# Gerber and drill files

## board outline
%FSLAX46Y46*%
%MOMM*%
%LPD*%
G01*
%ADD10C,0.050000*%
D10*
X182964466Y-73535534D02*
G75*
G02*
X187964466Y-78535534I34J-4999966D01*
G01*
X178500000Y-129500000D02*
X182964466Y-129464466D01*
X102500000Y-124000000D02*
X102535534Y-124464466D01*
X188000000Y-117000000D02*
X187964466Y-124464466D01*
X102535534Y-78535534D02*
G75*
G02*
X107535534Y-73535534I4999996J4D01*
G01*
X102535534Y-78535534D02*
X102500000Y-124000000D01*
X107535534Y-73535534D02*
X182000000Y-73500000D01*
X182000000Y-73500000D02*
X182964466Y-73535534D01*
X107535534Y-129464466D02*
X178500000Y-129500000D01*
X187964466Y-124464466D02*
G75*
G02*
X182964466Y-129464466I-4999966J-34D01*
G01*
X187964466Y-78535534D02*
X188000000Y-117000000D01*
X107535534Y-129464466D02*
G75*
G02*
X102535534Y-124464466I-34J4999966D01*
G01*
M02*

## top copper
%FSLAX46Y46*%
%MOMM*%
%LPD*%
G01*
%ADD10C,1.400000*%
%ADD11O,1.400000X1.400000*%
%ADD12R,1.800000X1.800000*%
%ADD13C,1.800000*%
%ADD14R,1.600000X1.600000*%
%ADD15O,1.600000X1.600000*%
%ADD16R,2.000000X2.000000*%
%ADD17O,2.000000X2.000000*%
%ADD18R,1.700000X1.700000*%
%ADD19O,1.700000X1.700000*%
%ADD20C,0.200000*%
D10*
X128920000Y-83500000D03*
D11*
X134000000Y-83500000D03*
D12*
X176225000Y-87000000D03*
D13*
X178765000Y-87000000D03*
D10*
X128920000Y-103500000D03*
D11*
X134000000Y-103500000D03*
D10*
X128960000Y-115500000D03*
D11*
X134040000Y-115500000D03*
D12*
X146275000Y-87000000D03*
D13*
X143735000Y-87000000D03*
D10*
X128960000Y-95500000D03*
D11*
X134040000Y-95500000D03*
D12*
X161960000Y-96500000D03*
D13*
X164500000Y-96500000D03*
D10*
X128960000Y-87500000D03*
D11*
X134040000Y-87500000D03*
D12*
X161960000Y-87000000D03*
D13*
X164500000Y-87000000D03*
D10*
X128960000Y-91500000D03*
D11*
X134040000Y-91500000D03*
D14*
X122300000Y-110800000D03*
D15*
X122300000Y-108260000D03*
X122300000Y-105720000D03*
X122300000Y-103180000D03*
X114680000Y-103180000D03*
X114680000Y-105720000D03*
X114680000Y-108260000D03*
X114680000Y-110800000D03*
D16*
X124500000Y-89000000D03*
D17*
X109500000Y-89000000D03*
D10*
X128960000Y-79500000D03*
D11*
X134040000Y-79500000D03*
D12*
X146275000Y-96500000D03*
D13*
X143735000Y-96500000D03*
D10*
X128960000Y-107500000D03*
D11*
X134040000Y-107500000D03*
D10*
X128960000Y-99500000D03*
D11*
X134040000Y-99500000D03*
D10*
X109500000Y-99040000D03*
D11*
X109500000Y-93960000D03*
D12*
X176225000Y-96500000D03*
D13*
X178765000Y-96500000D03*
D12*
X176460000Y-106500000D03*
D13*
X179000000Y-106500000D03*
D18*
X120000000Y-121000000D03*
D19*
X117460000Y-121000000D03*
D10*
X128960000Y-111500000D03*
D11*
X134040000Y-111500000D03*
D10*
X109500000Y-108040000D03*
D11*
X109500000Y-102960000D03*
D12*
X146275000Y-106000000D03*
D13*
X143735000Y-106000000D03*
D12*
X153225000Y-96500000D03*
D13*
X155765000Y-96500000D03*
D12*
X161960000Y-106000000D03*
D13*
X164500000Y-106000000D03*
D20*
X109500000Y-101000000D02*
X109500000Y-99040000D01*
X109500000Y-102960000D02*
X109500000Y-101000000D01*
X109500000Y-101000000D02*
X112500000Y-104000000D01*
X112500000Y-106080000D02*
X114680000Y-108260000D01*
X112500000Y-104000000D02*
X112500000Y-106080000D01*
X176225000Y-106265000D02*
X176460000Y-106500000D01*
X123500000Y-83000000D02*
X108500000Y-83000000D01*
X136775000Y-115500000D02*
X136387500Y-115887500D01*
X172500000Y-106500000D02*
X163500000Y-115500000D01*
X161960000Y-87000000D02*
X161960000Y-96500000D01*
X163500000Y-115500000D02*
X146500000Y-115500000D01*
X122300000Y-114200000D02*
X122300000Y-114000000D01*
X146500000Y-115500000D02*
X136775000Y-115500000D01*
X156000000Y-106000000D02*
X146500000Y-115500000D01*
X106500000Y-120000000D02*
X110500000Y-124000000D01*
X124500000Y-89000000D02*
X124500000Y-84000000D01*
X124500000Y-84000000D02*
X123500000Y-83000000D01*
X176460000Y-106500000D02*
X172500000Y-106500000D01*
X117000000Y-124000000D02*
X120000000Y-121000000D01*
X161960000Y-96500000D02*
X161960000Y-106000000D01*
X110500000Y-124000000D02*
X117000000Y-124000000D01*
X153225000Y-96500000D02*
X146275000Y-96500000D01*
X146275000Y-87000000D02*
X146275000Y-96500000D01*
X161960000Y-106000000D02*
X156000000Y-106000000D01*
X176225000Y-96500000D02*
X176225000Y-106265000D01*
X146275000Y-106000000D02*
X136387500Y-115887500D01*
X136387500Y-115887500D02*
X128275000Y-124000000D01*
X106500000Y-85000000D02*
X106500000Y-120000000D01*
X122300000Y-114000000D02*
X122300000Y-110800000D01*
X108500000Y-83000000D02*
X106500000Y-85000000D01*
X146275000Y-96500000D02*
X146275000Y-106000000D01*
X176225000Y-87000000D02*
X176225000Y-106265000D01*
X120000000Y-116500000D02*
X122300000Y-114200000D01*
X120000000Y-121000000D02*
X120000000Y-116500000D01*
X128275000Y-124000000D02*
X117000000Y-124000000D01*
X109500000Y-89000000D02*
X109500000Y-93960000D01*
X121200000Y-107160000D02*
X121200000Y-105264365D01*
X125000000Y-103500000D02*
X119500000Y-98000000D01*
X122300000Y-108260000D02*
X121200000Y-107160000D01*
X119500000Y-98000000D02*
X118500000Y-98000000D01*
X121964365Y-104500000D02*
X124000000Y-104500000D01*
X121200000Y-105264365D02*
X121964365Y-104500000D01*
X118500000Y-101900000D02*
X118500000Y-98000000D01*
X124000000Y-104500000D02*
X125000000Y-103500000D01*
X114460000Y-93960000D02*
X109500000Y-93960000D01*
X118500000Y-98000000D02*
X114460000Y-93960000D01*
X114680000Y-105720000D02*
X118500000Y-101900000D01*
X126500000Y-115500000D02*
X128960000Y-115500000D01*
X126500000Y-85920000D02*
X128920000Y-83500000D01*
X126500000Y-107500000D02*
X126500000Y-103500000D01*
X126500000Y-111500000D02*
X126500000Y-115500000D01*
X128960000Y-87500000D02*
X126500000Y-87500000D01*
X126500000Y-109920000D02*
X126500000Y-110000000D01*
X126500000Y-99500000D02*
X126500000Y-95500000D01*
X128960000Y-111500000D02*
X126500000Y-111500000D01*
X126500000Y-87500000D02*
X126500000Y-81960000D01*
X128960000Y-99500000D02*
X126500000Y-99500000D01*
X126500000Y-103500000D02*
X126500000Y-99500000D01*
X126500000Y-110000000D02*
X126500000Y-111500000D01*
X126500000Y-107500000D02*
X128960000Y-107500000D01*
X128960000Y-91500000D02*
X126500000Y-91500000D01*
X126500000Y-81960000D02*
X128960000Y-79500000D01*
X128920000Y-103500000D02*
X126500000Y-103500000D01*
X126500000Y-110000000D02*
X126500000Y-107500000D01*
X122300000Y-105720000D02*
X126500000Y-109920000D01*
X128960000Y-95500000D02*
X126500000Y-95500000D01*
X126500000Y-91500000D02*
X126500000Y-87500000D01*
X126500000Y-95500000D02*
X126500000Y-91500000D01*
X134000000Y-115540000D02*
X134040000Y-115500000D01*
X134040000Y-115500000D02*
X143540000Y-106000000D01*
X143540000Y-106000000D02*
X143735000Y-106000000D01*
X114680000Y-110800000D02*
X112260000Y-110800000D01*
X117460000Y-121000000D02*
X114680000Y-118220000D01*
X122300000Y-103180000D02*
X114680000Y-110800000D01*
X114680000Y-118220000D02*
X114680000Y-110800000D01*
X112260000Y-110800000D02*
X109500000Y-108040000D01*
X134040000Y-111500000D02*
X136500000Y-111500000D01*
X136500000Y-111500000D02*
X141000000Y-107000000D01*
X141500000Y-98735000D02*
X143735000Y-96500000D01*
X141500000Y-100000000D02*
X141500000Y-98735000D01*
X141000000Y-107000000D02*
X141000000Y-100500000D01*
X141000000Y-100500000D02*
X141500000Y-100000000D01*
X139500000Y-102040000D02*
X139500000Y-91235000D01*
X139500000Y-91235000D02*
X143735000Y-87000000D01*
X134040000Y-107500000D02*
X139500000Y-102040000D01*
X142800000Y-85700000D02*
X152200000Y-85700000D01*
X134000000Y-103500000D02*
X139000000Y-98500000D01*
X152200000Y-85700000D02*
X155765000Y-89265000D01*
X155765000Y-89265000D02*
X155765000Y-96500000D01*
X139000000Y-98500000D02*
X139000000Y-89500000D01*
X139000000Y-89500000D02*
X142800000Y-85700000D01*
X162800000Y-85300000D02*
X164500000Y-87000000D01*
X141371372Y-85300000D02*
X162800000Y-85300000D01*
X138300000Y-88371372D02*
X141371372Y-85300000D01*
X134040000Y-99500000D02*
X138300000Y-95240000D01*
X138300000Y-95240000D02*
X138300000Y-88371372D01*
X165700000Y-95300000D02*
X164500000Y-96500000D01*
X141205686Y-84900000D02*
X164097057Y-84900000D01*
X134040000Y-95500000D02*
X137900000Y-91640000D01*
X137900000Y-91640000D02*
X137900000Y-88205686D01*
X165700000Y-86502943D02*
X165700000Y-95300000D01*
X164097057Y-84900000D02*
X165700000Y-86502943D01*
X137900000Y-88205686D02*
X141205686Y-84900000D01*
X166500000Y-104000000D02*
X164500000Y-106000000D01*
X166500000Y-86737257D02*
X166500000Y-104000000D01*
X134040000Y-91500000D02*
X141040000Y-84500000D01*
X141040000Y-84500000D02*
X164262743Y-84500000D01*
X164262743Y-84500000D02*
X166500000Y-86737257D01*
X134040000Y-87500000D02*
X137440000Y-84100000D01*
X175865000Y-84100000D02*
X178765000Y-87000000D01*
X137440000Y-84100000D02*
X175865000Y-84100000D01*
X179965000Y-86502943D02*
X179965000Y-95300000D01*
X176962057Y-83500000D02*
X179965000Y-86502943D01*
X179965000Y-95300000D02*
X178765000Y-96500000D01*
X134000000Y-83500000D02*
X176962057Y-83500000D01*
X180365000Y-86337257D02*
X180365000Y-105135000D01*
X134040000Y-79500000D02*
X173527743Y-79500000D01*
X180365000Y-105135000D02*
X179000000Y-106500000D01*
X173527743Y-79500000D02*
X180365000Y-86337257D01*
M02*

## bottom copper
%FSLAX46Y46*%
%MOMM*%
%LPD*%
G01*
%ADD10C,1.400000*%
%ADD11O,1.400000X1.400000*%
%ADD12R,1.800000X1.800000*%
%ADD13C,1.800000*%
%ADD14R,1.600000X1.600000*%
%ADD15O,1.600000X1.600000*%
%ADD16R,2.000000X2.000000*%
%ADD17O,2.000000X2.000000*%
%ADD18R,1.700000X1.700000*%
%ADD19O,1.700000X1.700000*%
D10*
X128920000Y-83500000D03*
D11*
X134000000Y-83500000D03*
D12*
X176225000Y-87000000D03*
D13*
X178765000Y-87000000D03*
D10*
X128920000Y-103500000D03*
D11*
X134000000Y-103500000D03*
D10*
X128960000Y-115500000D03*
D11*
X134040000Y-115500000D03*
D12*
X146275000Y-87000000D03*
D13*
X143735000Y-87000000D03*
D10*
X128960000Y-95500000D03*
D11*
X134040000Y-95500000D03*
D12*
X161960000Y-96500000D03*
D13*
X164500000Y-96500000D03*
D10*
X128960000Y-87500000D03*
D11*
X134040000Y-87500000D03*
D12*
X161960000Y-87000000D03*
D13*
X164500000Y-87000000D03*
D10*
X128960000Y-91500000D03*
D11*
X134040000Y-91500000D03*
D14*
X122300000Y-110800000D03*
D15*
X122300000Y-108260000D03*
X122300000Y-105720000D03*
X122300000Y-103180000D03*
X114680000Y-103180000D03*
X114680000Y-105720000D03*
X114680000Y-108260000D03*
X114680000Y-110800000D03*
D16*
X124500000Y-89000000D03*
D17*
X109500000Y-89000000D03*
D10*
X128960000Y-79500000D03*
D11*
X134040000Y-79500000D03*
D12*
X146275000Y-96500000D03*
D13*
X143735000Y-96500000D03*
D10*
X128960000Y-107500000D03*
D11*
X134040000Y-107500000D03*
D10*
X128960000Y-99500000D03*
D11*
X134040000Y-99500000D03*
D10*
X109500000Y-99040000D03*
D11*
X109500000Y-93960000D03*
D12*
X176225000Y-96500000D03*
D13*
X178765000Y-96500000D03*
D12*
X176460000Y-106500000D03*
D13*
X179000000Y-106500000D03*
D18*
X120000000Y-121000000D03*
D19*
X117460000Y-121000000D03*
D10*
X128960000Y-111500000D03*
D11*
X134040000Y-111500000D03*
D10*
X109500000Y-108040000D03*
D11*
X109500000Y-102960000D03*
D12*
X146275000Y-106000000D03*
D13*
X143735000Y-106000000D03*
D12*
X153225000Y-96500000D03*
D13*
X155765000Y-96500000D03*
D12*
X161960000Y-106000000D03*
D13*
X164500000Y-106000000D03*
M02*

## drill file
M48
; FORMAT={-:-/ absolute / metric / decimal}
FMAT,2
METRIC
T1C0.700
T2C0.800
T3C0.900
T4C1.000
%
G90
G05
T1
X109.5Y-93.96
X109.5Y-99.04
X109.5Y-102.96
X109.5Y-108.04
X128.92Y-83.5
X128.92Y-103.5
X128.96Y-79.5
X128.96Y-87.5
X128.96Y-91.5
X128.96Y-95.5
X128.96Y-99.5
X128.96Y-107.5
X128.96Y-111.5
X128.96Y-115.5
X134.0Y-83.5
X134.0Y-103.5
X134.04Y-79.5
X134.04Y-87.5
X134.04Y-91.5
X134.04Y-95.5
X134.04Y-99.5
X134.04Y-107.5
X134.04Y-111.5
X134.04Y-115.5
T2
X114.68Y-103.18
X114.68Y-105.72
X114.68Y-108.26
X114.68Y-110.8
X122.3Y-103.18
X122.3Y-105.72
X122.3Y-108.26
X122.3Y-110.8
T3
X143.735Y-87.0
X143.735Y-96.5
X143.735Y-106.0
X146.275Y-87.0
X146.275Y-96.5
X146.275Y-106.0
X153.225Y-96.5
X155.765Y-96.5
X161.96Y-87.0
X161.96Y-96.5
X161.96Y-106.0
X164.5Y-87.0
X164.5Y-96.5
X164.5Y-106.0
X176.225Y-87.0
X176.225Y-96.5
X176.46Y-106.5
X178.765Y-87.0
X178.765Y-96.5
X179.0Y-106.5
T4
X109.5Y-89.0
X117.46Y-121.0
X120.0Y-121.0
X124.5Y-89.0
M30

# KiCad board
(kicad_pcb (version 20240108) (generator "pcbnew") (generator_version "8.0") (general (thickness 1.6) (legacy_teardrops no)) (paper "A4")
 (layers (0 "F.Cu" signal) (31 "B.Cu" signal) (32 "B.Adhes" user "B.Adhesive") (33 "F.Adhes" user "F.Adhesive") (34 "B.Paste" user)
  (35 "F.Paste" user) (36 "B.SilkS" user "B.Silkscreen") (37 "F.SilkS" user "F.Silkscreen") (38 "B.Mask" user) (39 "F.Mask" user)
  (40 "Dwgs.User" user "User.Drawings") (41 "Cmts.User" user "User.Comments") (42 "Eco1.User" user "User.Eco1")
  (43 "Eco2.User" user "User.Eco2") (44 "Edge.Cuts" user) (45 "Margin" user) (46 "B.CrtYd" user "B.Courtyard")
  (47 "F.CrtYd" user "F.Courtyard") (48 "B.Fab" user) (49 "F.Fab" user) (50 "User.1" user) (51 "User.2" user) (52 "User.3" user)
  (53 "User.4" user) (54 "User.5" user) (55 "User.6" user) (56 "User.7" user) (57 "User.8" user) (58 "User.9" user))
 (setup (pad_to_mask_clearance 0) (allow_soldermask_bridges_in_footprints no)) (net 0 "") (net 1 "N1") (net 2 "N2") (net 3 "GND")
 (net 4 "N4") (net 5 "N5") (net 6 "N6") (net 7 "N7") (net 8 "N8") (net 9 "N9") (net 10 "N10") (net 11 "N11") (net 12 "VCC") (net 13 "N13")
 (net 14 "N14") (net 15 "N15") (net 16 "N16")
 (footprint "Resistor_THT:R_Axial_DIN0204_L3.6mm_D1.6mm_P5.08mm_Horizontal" (layer "F.Cu") (at 128.92 83.5)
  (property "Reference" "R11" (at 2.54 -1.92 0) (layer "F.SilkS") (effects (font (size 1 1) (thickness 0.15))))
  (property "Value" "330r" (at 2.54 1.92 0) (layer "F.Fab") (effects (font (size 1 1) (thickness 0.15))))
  (pad "1" thru_hole circle (at 0 0) (size 1.4 1.4) (drill 0.7) (layers "*.Cu" "*.Mask") (remove_unused_layers no) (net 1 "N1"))
  (pad "2" thru_hole oval (at 5.08 0) (size 1.4 1.4) (drill 0.7) (layers "*.Cu" "*.Mask") (remove_unused_layers no) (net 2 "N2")))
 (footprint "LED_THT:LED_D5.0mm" (layer "F.Cu") (at 176.225 87)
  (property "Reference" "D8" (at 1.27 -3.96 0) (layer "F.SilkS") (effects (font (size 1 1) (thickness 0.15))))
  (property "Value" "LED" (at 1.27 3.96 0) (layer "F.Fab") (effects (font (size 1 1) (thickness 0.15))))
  (pad "1" thru_hole rect (at 0 0) (size 1.8 1.8) (drill 0.9) (layers "*.Cu" "*.Mask") (remove_unused_layers no) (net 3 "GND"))
  (pad "2" thru_hole circle (at 2.54 0) (size 1.8 1.8) (drill 0.9) (layers "*.Cu" "*.Mask") (remove_unused_layers no) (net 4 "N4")))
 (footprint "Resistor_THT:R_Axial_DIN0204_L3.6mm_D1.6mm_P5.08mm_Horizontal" (layer "F.Cu") (at 128.92 103.5)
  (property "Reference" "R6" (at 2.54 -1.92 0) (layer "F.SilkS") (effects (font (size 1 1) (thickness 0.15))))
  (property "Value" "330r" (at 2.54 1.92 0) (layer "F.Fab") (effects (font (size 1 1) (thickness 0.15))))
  (pad "1" thru_hole circle (at 0 0) (size 1.4 1.4) (drill 0.7) (layers "*.Cu" "*.Mask") (remove_unused_layers no) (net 1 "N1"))
  (pad "2" thru_hole oval (at 5.08 0) (size 1.4 1.4) (drill 0.7) (layers "*.Cu" "*.Mask") (remove_unused_layers no) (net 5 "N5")))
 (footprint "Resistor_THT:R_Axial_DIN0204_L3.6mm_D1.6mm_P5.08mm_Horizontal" (layer "F.Cu") (at 128.96 115.5)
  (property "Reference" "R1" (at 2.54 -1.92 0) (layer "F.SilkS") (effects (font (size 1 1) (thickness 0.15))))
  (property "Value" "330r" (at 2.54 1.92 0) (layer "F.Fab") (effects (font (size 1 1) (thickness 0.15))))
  (pad "1" thru_hole circle (at 0 0) (size 1.4 1.4) (drill 0.7) (layers "*.Cu" "*.Mask") (remove_unused_layers no) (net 1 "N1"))
  (pad "2" thru_hole oval (at 5.08 0) (size 1.4 1.4) (drill 0.7) (layers "*.Cu" "*.Mask") (remove_unused_layers no) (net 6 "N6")))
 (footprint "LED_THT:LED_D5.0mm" (layer "F.Cu") (at 146.275 87 180)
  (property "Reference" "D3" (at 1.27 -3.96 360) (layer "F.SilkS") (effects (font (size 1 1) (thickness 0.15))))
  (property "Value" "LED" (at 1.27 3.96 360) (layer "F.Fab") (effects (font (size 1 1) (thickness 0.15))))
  (pad "1" thru_hole rect (at 0 0 180) (size 1.8 1.8) (drill 0.9) (layers "*.Cu" "*.Mask") (remove_unused_layers no) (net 3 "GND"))
  (pad "2" thru_hole circle (at 2.54 0 180) (size 1.8 1.8) (drill 0.9) (layers "*.Cu" "*.Mask") (remove_unused_layers no) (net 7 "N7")))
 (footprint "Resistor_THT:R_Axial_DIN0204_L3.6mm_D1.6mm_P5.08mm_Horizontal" (layer "F.Cu") (at 128.96 95.5)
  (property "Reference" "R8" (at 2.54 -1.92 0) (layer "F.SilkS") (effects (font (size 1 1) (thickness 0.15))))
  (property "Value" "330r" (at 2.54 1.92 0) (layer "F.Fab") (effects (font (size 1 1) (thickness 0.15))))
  (pad "1" thru_hole circle (at 0 0) (size 1.4 1.4) (drill 0.7) (layers "*.Cu" "*.Mask") (remove_unused_layers no) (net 1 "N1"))
  (pad "2" thru_hole oval (at 5.08 0) (size 1.4 1.4) (drill 0.7) (layers "*.Cu" "*.Mask") (remove_unused_layers no) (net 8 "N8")))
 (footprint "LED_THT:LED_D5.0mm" (layer "F.Cu") (at 161.96 96.5)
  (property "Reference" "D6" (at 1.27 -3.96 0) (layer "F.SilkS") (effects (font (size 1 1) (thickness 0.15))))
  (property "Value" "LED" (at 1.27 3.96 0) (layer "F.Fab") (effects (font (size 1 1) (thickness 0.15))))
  (pad "1" thru_hole rect (at 0 0) (size 1.8 1.8) (drill 0.9) (layers "*.Cu" "*.Mask") (remove_unused_layers no) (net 3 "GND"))
  (pad "2" thru_hole circle (at 2.54 0) (size 1.8 1.8) (drill 0.9) (layers "*.Cu" "*.Mask") (remove_unused_layers no) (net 8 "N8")))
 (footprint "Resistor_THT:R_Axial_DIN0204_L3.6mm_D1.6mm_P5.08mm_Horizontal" (layer "F.Cu") (at 128.96 87.5)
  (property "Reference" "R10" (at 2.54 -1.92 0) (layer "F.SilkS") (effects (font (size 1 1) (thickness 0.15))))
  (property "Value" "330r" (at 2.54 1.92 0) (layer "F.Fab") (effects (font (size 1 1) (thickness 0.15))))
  (pad "1" thru_hole circle (at 0 0) (size 1.4 1.4) (drill 0.7) (layers "*.Cu" "*.Mask") (remove_unused_layers no) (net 1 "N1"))
  (pad "2" thru_hole oval (at 5.08 0) (size 1.4 1.4) (drill 0.7) (layers "*.Cu" "*.Mask") (remove_unused_layers no) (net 4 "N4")))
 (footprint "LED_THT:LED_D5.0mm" (layer "F.Cu") (at 161.96 87)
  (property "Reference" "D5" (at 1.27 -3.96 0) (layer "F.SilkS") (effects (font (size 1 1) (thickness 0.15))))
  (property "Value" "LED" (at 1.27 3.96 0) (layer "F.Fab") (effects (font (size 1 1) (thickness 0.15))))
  (pad "1" thru_hole rect (at 0 0) (size 1.8 1.8) (drill 0.9) (layers "*.Cu" "*.Mask") (remove_unused_layers no) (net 3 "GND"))
  (pad "2" thru_hole circle (at 2.54 0) (size 1.8 1.8) (drill 0.9) (layers "*.Cu" "*.Mask") (remove_unused_layers no) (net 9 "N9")))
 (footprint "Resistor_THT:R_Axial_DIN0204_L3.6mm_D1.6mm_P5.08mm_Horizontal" (layer "F.Cu") (at 128.96 91.5)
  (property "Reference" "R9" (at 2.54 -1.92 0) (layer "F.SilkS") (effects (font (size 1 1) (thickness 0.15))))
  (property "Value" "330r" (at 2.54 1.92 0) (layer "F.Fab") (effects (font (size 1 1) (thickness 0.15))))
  (pad "1" thru_hole circle (at 0 0) (size 1.4 1.4) (drill 0.7) (layers "*.Cu" "*.Mask") (remove_unused_layers no) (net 1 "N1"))
  (pad "2" thru_hole oval (at 5.08 0) (size 1.4 1.4) (drill 0.7) (layers "*.Cu" "*.Mask") (remove_unused_layers no) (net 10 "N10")))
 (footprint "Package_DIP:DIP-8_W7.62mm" (layer "F.Cu") (at 122.3 110.8 180)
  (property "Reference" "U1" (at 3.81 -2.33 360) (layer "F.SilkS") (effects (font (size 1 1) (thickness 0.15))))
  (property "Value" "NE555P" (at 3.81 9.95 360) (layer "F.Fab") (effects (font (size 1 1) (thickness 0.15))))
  (pad "1" thru_hole rect (at 0 0 180) (size 1.6 1.6) (drill 0.8) (layers "*.Cu" "*.Mask") (remove_unused_layers no) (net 3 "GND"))
  (pad "2" thru_hole oval (at 0 2.54 180) (size 1.6 1.6) (drill 0.8) (layers "*.Cu" "*.Mask") (remove_unused_layers no) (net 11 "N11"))
  (pad "3" thru_hole oval (at 0 5.08 180) (size 1.6 1.6) (drill 0.8) (layers "*.Cu" "*.Mask") (remove_unused_layers no) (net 1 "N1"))
  (pad "4" thru_hole oval (at 0 7.62 180) (size 1.6 1.6) (drill 0.8) (layers "*.Cu" "*.Mask") (remove_unused_layers no) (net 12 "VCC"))
  (pad "5" thru_hole oval (at 7.62 7.62 180) (size 1.6 1.6) (drill 0.8) (layers "*.Cu" "*.Mask") (remove_unused_layers no) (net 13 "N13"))
  (pad "6" thru_hole oval (at 7.62 5.08 180) (size 1.6 1.6) (drill 0.8) (layers "*.Cu" "*.Mask") (remove_unused_layers no) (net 11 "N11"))
  (pad "7" thru_hole oval (at 7.62 2.54 180) (size 1.6 1.6) (drill 0.8) (layers "*.Cu" "*.Mask") (remove_unused_layers no) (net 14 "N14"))
  (pad "8" thru_hole oval (at 7.62 0 180) (size 1.6 1.6) (drill 0.8) (layers "*.Cu" "*.Mask") (remove_unused_layers no) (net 12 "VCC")))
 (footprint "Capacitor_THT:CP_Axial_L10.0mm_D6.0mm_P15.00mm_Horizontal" (layer "F.Cu") (at 124.5 89 180)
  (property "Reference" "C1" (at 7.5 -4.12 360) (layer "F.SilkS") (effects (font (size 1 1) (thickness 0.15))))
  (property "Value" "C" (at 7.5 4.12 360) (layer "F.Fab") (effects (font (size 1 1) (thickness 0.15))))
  (pad "1" thru_hole rect (at 0 0 180) (size 2 2) (drill 1) (layers "*.Cu" "*.Mask") (remove_unused_layers no) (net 3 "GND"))
  (pad "2" thru_hole oval (at 15 0 180) (size 2 2) (drill 1) (layers "*.Cu" "*.Mask") (remove_unused_layers no) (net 11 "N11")))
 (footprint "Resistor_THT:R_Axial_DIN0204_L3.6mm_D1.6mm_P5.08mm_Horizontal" (layer "F.Cu") (at 128.96 79.5)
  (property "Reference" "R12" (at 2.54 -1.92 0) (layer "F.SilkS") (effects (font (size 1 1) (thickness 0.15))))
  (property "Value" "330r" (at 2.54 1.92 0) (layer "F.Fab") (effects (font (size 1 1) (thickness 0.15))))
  (pad "1" thru_hole circle (at 0 0) (size 1.4 1.4) (drill 0.7) (layers "*.Cu" "*.Mask") (remove_unused_layers no) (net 1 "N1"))
  (pad "2" thru_hole oval (at 5.08 0) (size 1.4 1.4) (drill 0.7) (layers "*.Cu" "*.Mask") (remove_unused_layers no) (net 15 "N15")))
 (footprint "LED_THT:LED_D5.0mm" (layer "F.Cu") (at 146.275 96.5 180)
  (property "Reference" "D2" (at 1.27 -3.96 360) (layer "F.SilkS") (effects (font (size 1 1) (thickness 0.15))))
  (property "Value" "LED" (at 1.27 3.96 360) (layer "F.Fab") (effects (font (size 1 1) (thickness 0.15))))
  (pad "1" thru_hole rect (at 0 0 180) (size 1.8 1.8) (drill 0.9) (layers "*.Cu" "*.Mask") (remove_unused_layers no) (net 3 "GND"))
  (pad "2" thru_hole circle (at 2.54 0 180) (size 1.8 1.8) (drill 0.9) (layers "*.Cu" "*.Mask") (remove_unused_layers no) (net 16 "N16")))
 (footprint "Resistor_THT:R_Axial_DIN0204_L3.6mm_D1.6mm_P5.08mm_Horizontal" (layer "F.Cu") (at 128.96 107.5)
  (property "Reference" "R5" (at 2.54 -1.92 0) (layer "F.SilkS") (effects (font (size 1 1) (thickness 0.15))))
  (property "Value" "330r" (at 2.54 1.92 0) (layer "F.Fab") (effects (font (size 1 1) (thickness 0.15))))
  (pad "1" thru_hole circle (at 0 0) (size 1.4 1.4) (drill 0.7) (layers "*.Cu" "*.Mask") (remove_unused_layers no) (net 1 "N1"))
  (pad "2" thru_hole oval (at 5.08 0) (size 1.4 1.4) (drill 0.7) (layers "*.Cu" "*.Mask") (remove_unused_layers no) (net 7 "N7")))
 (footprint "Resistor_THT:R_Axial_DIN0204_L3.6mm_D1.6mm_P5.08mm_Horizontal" (layer "F.Cu") (at 128.96 99.5)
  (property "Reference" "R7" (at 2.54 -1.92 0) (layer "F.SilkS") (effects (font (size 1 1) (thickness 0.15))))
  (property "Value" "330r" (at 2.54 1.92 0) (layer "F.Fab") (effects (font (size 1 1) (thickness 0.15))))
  (pad "1" thru_hole circle (at 0 0) (size 1.4 1.4) (drill 0.7) (layers "*.Cu" "*.Mask") (remove_unused_layers no) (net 1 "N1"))
  (pad "2" thru_hole oval (at 5.08 0) (size 1.4 1.4) (drill 0.7) (layers "*.Cu" "*.Mask") (remove_unused_layers no) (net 9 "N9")))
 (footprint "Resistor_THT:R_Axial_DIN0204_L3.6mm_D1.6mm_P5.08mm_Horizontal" (layer "F.Cu") (at 109.5 99.04 90)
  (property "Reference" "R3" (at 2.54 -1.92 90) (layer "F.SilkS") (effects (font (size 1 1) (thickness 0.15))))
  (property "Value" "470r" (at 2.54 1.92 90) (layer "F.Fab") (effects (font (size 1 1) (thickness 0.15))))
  (pad "1" thru_hole circle (at 0 0 90) (size 1.4 1.4) (drill 0.7) (layers "*.Cu" "*.Mask") (remove_unused_layers no) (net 14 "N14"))
  (pad "2" thru_hole oval (at 5.08 0 90) (size 1.4 1.4) (drill 0.7) (layers "*.Cu" "*.Mask") (remove_unused_layers no) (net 11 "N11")))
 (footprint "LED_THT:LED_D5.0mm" (layer "F.Cu") (at 176.225 96.5)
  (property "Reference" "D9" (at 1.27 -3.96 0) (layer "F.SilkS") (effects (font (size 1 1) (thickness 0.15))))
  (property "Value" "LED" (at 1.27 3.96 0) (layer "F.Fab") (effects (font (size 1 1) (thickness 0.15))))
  (pad "1" thru_hole rect (at 0 0) (size 1.8 1.8) (drill 0.9) (layers "*.Cu" "*.Mask") (remove_unused_layers no) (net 3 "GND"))
  (pad "2" thru_hole circle (at 2.54 0) (size 1.8 1.8) (drill 0.9) (layers "*.Cu" "*.Mask") (remove_unused_layers no) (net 2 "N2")))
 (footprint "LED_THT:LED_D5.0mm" (layer "F.Cu") (at 176.46 106.5)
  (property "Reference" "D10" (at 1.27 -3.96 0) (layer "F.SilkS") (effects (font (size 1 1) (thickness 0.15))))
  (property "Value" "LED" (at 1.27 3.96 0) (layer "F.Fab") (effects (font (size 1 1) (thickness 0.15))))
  (pad "1" thru_hole rect (at 0 0) (size 1.8 1.8) (drill 0.9) (layers "*.Cu" "*.Mask") (remove_unused_layers no) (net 3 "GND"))
  (pad "2" thru_hole circle (at 2.54 0) (size 1.8 1.8) (drill 0.9) (layers "*.Cu" "*.Mask") (remove_unused_layers no) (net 15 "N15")))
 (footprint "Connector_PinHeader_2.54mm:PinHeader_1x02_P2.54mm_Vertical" (layer "F.Cu") (at 120 121 -90)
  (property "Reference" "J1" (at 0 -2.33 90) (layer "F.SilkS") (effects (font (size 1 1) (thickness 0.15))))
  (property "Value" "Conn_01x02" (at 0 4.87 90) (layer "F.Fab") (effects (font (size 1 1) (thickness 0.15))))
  (pad "1" thru_hole rect (at 0 0 270) (size 1.7 1.7) (drill 1) (layers "*.Cu" "*.Mask") (remove_unused_layers no) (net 3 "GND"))
  (pad "2" thru_hole oval (at 0 2.54 270) (size 1.7 1.7) (drill 1) (layers "*.Cu" "*.Mask") (remove_unused_layers no) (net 12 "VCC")))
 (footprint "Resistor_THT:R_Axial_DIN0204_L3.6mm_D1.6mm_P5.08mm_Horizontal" (layer "F.Cu") (at 128.96 111.5)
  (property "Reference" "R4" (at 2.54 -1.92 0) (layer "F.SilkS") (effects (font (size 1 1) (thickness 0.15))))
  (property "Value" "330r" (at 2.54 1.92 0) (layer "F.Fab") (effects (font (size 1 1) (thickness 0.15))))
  (pad "1" thru_hole circle (at 0 0) (size 1.4 1.4) (drill 0.7) (layers "*.Cu" "*.Mask") (remove_unused_layers no) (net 1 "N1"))
  (pad "2" thru_hole oval (at 5.08 0) (size 1.4 1.4) (drill 0.7) (layers "*.Cu" "*.Mask") (remove_unused_layers no) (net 16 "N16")))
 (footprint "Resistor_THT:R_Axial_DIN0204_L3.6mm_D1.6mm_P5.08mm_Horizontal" (layer "F.Cu") (at 109.5 108.04 90)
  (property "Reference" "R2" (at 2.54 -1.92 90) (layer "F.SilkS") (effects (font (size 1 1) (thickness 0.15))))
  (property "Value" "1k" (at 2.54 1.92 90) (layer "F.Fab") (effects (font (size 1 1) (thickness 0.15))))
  (pad "1" thru_hole circle (at 0 0 90) (size 1.4 1.4) (drill 0.7) (layers "*.Cu" "*.Mask") (remove_unused_layers no) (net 12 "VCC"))
  (pad "2" thru_hole oval (at 5.08 0 90) (size 1.4 1.4) (drill 0.7) (layers "*.Cu" "*.Mask") (remove_unused_layers no) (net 14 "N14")))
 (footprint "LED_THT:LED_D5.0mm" (layer "F.Cu") (at 146.275 106 180)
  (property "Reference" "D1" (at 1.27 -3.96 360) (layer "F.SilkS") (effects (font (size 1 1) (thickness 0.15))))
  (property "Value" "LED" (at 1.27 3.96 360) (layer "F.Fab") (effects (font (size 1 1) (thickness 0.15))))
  (pad "1" thru_hole rect (at 0 0 180) (size 1.8 1.8) (drill 0.9) (layers "*.Cu" "*.Mask") (remove_unused_layers no) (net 3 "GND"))
  (pad "2" thru_hole circle (at 2.54 0 180) (size 1.8 1.8) (drill 0.9) (layers "*.Cu" "*.Mask") (remove_unused_layers no) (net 6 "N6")))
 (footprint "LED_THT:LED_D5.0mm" (layer "F.Cu") (at 153.225 96.5)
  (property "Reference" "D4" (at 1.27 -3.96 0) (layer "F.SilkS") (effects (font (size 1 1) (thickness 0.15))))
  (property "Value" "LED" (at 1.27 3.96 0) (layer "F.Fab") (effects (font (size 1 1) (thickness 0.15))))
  (pad "1" thru_hole rect (at 0 0) (size 1.8 1.8) (drill 0.9) (layers "*.Cu" "*.Mask") (remove_unused_layers no) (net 3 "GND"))
  (pad "2" thru_hole circle (at 2.54 0) (size 1.8 1.8) (drill 0.9) (layers "*.Cu" "*.Mask") (remove_unused_layers no) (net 5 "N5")))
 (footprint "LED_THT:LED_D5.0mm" (layer "F.Cu") (at 161.96 106)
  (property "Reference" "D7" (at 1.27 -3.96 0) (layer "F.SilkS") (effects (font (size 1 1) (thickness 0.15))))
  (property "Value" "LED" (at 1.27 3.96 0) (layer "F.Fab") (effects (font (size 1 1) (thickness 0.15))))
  (pad "1" thru_hole rect (at 0 0) (size 1.8 1.8) (drill 0.9) (layers "*.Cu" "*.Mask") (remove_unused_layers no) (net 3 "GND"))
  (pad "2" thru_hole circle (at 2.54 0) (size 1.8 1.8) (drill 0.9) (layers "*.Cu" "*.Mask") (remove_unused_layers no) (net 10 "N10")))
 (gr_arc (start 182.964466 73.535534) (mid 186.5 75) (end 187.964466 78.535534) (stroke (width 0.05) (type default)) (layer "Edge.Cuts"))
 (gr_line (start 178.5 129.5) (end 182.964466 129.464466) (stroke (width 0.05) (type default)) (layer "Edge.Cuts"))
 (gr_line (start 102.5 124) (end 102.535534 124.464466) (stroke (width 0.05) (type default)) (layer "Edge.Cuts"))
 (gr_line (start 188 117) (end 187.964466 124.464466) (stroke (width 0.05) (type default)) (layer "Edge.Cuts"))
 (gr_arc (start 102.535534 78.535534) (mid 104 75) (end 107.535534 73.535534) (stroke (width 0.05) (type default)) (layer "Edge.Cuts"))
 (gr_line (start 102.535534 78.535534) (end 102.5 124) (stroke (width 0.05) (type default)) (layer "Edge.Cuts"))
 (gr_line (start 107.535534 73.535534) (end 182 73.5) (stroke (width 0.05) (type default)) (layer "Edge.Cuts"))
 (gr_line (start 182 73.5) (end 182.964466 73.535534) (stroke (width 0.05) (type default)) (layer "Edge.Cuts"))
 (gr_line (start 107.535534 129.464466) (end 178.5 129.5) (stroke (width 0.05) (type default)) (layer "Edge.Cuts"))
 (gr_arc (start 187.964466 124.464466) (mid 186.5 128) (end 182.964466 129.464466) (stroke (width 0.05) (type default)) (layer "Edge.Cuts"))
 (gr_line (start 187.964466 78.535534) (end 188 117) (stroke (width 0.05) (type default)) (layer "Edge.Cuts"))
 (gr_arc (start 107.535534 129.464466) (mid 104 128) (end 102.535534 124.464466) (stroke (width 0.05) (type default)) (layer "Edge.Cuts"))
 (segment (start 109.5 101) (end 109.5 99.04) (width 0.2) (layer "F.Cu") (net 14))
 (segment (start 109.5 102.96) (end 109.5 101) (width 0.2) (layer "F.Cu") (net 14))
 (segment (start 109.5 101) (end 112.5 104) (width 0.2) (layer "F.Cu") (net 14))
 (segment (start 112.5 106.08) (end 114.68 108.26) (width 0.2) (layer "F.Cu") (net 14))
 (segment (start 112.5 104) (end 112.5 106.08) (width 0.2) (layer "F.Cu") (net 14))
 (segment (start 176.225 106.265) (end 176.46 106.5) (width 0.2) (layer "F.Cu") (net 3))
 (segment (start 123.5 83) (end 108.5 83) (width 0.2) (layer "F.Cu") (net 3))
 (segment (start 136.775 115.5) (end 136.3875 115.8875) (width 0.2) (layer "F.Cu") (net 3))
 (segment (start 172.5 106.5) (end 163.5 115.5) (width 0.2) (layer "F.Cu") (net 3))
 (segment (start 161.96 87) (end 161.96 96.5) (width 0.2) (layer "F.Cu") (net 3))
 (segment (start 163.5 115.5) (end 146.5 115.5) (width 0.2) (layer "F.Cu") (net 3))
 (segment (start 122.3 114.2) (end 122.3 114) (width 0.2) (layer "F.Cu") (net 3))
 (segment (start 146.5 115.5) (end 136.775 115.5) (width 0.2) (layer "F.Cu") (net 3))
 (segment (start 156 106) (end 146.5 115.5) (width 0.2) (layer "F.Cu") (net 3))
 (segment (start 106.5 120) (end 110.5 124) (width 0.2) (layer "F.Cu") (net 3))
 (segment (start 124.5 89) (end 124.5 84) (width 0.2) (layer "F.Cu") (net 3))
 (segment (start 124.5 84) (end 123.5 83) (width 0.2) (layer "F.Cu") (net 3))
 (segment (start 176.46 106.5) (end 172.5 106.5) (width 0.2) (layer "F.Cu") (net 3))
 (segment (start 117 124) (end 120 121) (width 0.2) (layer "F.Cu") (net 3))
 (segment (start 161.96 96.5) (end 161.96 106) (width 0.2) (layer "F.Cu") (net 3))
 (segment (start 110.5 124) (end 117 124) (width 0.2) (layer "F.Cu") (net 3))
 (segment (start 153.225 96.5) (end 146.275 96.5) (width 0.2) (layer "F.Cu") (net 3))
 (segment (start 146.275 87) (end 146.275 96.5) (width 0.2) (layer "F.Cu") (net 3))
 (segment (start 161.96 106) (end 156 106) (width 0.2) (layer "F.Cu") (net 3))
 (segment (start 176.225 96.5) (end 176.225 106.265) (width 0.2) (layer "F.Cu") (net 3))
 (segment (start 146.275 106) (end 136.3875 115.8875) (width 0.2) (layer "F.Cu") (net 3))
 (segment (start 136.3875 115.8875) (end 128.275 124) (width 0.2) (layer "F.Cu") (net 3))
 (segment (start 106.5 85) (end 106.5 120) (width 0.2) (layer "F.Cu") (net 3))
 (segment (start 122.3 114) (end 122.3 110.8) (width 0.2) (layer "F.Cu") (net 3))
 (segment (start 108.5 83) (end 106.5 85) (width 0.2) (layer "F.Cu") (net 3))
 (segment (start 146.275 96.5) (end 146.275 106) (width 0.2) (layer "F.Cu") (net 3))
 (segment (start 176.225 87) (end 176.225 106.265) (width 0.2) (layer "F.Cu") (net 3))
 (segment (start 120 116.5) (end 122.3 114.2) (width 0.2) (layer "F.Cu") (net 3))
 (segment (start 120 121) (end 120 116.5) (width 0.2) (layer "F.Cu") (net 3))
 (segment (start 128.275 124) (end 117 124) (width 0.2) (layer "F.Cu") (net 3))
 (segment (start 109.5 89) (end 109.5 93.96) (width 0.2) (layer "F.Cu") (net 11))
 (segment (start 121.2 107.16) (end 121.2 105.264365) (width 0.2) (layer "F.Cu") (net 11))
 (segment (start 125 103.5) (end 119.5 98) (width 0.2) (layer "F.Cu") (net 11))
 (segment (start 122.3 108.26) (end 121.2 107.16) (width 0.2) (layer "F.Cu") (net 11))
 (segment (start 119.5 98) (end 118.5 98) (width 0.2) (layer "F.Cu") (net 11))
 (segment (start 121.964365 104.5) (end 124 104.5) (width 0.2) (layer "F.Cu") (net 11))
 (segment (start 121.2 105.264365) (end 121.964365 104.5) (width 0.2) (layer "F.Cu") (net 11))
 (segment (start 118.5 101.9) (end 118.5 98) (width 0.2) (layer "F.Cu") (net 11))
 (segment (start 124 104.5) (end 125 103.5) (width 0.2) (layer "F.Cu") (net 11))
 (segment (start 114.46 93.96) (end 109.5 93.96) (width 0.2) (layer "F.Cu") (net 11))
 (segment (start 118.5 98) (end 114.46 93.96) (width 0.2) (layer "F.Cu") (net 11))
 (segment (start 114.68 105.72) (end 118.5 101.9) (width 0.2) (layer "F.Cu") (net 11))
 (segment (start 126.5 115.5) (end 128.96 115.5) (width 0.2) (layer "F.Cu") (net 1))
 (segment (start 126.5 85.92) (end 128.92 83.5) (width 0.2) (layer "F.Cu") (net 1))
 (segment (start 126.5 107.5) (end 126.5 103.5) (width 0.2) (layer "F.Cu") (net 1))
 (segment (start 126.5 111.5) (end 126.5 115.5) (width 0.2) (layer "F.Cu") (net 1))
 (segment (start 128.96 87.5) (end 126.5 87.5) (width 0.2) (layer "F.Cu") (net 1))
 (segment (start 126.5 109.92) (end 126.5 110) (width 0.2) (layer "F.Cu") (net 1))
 (segment (start 126.5 99.5) (end 126.5 95.5) (width 0.2) (layer "F.Cu") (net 1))
 (segment (start 128.96 111.5) (end 126.5 111.5) (width 0.2) (layer "F.Cu") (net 1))
 (segment (start 126.5 87.5) (end 126.5 81.96) (width 0.2) (layer "F.Cu") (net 1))
 (segment (start 128.96 99.5) (end 126.5 99.5) (width 0.2) (layer "F.Cu") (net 1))
 (segment (start 126.5 103.5) (end 126.5 99.5) (width 0.2) (layer "F.Cu") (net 1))
 (segment (start 126.5 110) (end 126.5 111.5) (width 0.2) (layer "F.Cu") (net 1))
 (segment (start 126.5 107.5) (end 128.96 107.5) (width 0.2) (layer "F.Cu") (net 1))
 (segment (start 128.96 91.5) (end 126.5 91.5) (width 0.2) (layer "F.Cu") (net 1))
 (segment (start 126.5 81.96) (end 128.96 79.5) (width 0.2) (layer "F.Cu") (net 1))
 (segment (start 128.92 103.5) (end 126.5 103.5) (width 0.2) (layer "F.Cu") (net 1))
 (segment (start 126.5 110) (end 126.5 107.5) (width 0.2) (layer "F.Cu") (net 1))
 (segment (start 122.3 105.72) (end 126.5 109.92) (width 0.2) (layer "F.Cu") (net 1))
 (segment (start 128.96 95.5) (end 126.5 95.5) (width 0.2) (layer "F.Cu") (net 1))
 (segment (start 126.5 91.5) (end 126.5 87.5) (width 0.2) (layer "F.Cu") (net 1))
 (segment (start 126.5 95.5) (end 126.5 91.5) (width 0.2) (layer "F.Cu") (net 1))
 (segment (start 134 115.54) (end 134.04 115.5) (width 0.2) (layer "F.Cu") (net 6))
 (segment (start 134.04 115.5) (end 143.54 106) (width 0.2) (layer "F.Cu") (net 6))
 (segment (start 143.54 106) (end 143.735 106) (width 0.2) (layer "F.Cu") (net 6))
 (segment (start 114.68 110.8) (end 112.26 110.8) (width 0.2) (layer "F.Cu") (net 12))
 (segment (start 117.46 121) (end 114.68 118.22) (width 0.2) (layer "F.Cu") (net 12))
 (segment (start 122.3 103.18) (end 114.68 110.8) (width 0.2) (layer "F.Cu") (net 12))
 (segment (start 114.68 118.22) (end 114.68 110.8) (width 0.2) (layer "F.Cu") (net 12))
 (segment (start 112.26 110.8) (end 109.5 108.04) (width 0.2) (layer "F.Cu") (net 12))
 (segment (start 134.04 111.5) (end 136.5 111.5) (width 0.2) (layer "F.Cu") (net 16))
 (segment (start 136.5 111.5) (end 141 107) (width 0.2) (layer "F.Cu") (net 16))
 (segment (start 141.5 98.735) (end 143.735 96.5) (width 0.2) (layer "F.Cu") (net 16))
 (segment (start 141.5 100) (end 141.5 98.735) (width 0.2) (layer "F.Cu") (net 16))
 (segment (start 141 107) (end 141 100.5) (width 0.2) (layer "F.Cu") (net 16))
 (segment (start 141 100.5) (end 141.5 100) (width 0.2) (layer "F.Cu") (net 16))
 (segment (start 139.5 102.04) (end 139.5 91.235) (width 0.2) (layer "F.Cu") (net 7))
 (segment (start 139.5 91.235) (end 143.735 87) (width 0.2) (layer "F.Cu") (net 7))
 (segment (start 134.04 107.5) (end 139.5 102.04) (width 0.2) (layer "F.Cu") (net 7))
 (segment (start 142.8 85.7) (end 152.2 85.7) (width 0.2) (layer "F.Cu") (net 5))
 (segment (start 134 103.5) (end 139 98.5) (width 0.2) (layer "F.Cu") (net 5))
 (segment (start 152.2 85.7) (end 155.765 89.265) (width 0.2) (layer "F.Cu") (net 5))
 (segment (start 155.765 89.265) (end 155.765 96.5) (width 0.2) (layer "F.Cu") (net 5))
 (segment (start 139 98.5) (end 139 89.5) (width 0.2) (layer "F.Cu") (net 5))
 (segment (start 139 89.5) (end 142.8 85.7) (width 0.2) (layer "F.Cu") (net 5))
 (segment (start 162.8 85.3) (end 164.5 87) (width 0.2) (layer "F.Cu") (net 9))
 (segment (start 141.371372 85.3) (end 162.8 85.3) (width 0.2) (layer "F.Cu") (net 9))
 (segment (start 138.3 88.371372) (end 141.371372 85.3) (width 0.2) (layer "F.Cu") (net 9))
 (segment (start 134.04 99.5) (end 138.3 95.24) (width 0.2) (layer "F.Cu") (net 9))
 (segment (start 138.3 95.24) (end 138.3 88.371372) (width 0.2) (layer "F.Cu") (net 9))
 (segment (start 165.7 95.3) (end 164.5 96.5) (width 0.2) (layer "F.Cu") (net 8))
 (segment (start 141.205686 84.9) (end 164.097057 84.9) (width 0.2) (layer "F.Cu") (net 8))
 (segment (start 134.04 95.5) (end 137.9 91.64) (width 0.2) (layer "F.Cu") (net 8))
 (segment (start 137.9 91.64) (end 137.9 88.205686) (width 0.2) (layer "F.Cu") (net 8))
 (segment (start 165.7 86.502943) (end 165.7 95.3) (width 0.2) (layer "F.Cu") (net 8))
 (segment (start 164.097057 84.9) (end 165.7 86.502943) (width 0.2) (layer "F.Cu") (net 8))
 (segment (start 137.9 88.205686) (end 141.205686 84.9) (width 0.2) (layer "F.Cu") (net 8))
 (segment (start 166.5 104) (end 164.5 106) (width 0.2) (layer "F.Cu") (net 10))
 (segment (start 166.5 86.737257) (end 166.5 104) (width 0.2) (layer "F.Cu") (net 10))
 (segment (start 134.04 91.5) (end 141.04 84.5) (width 0.2) (layer "F.Cu") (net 10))
 (segment (start 141.04 84.5) (end 164.262743 84.5) (width 0.2) (layer "F.Cu") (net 10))
 (segment (start 164.262743 84.5) (end 166.5 86.737257) (width 0.2) (layer "F.Cu") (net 10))
 (segment (start 134.04 87.5) (end 137.44 84.1) (width 0.2) (layer "F.Cu") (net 4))
 (segment (start 175.865 84.1) (end 178.765 87) (width 0.2) (layer "F.Cu") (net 4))
 (segment (start 137.44 84.1) (end 175.865 84.1) (width 0.2) (layer "F.Cu") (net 4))
 (segment (start 179.965 86.502943) (end 179.965 95.3) (width 0.2) (layer "F.Cu") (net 2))
 (segment (start 176.962057 83.5) (end 179.965 86.502943) (width 0.2) (layer "F.Cu") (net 2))
 (segment (start 179.965 95.3) (end 178.765 96.5) (width 0.2) (layer "F.Cu") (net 2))
 (segment (start 134 83.5) (end 176.962057 83.5) (width 0.2) (layer "F.Cu") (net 2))
 (segment (start 180.365 86.337257) (end 180.365 105.135) (width 0.2) (layer "F.Cu") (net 15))
 (segment (start 134.04 79.5) (end 173.527743 79.5) (width 0.2) (layer "F.Cu") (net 15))
 (segment (start 180.365 105.135) (end 179 106.5) (width 0.2) (layer "F.Cu") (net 15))
 (segment (start 173.527743 79.5) (end 180.365 86.337257) (width 0.2) (layer "F.Cu") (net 15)))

